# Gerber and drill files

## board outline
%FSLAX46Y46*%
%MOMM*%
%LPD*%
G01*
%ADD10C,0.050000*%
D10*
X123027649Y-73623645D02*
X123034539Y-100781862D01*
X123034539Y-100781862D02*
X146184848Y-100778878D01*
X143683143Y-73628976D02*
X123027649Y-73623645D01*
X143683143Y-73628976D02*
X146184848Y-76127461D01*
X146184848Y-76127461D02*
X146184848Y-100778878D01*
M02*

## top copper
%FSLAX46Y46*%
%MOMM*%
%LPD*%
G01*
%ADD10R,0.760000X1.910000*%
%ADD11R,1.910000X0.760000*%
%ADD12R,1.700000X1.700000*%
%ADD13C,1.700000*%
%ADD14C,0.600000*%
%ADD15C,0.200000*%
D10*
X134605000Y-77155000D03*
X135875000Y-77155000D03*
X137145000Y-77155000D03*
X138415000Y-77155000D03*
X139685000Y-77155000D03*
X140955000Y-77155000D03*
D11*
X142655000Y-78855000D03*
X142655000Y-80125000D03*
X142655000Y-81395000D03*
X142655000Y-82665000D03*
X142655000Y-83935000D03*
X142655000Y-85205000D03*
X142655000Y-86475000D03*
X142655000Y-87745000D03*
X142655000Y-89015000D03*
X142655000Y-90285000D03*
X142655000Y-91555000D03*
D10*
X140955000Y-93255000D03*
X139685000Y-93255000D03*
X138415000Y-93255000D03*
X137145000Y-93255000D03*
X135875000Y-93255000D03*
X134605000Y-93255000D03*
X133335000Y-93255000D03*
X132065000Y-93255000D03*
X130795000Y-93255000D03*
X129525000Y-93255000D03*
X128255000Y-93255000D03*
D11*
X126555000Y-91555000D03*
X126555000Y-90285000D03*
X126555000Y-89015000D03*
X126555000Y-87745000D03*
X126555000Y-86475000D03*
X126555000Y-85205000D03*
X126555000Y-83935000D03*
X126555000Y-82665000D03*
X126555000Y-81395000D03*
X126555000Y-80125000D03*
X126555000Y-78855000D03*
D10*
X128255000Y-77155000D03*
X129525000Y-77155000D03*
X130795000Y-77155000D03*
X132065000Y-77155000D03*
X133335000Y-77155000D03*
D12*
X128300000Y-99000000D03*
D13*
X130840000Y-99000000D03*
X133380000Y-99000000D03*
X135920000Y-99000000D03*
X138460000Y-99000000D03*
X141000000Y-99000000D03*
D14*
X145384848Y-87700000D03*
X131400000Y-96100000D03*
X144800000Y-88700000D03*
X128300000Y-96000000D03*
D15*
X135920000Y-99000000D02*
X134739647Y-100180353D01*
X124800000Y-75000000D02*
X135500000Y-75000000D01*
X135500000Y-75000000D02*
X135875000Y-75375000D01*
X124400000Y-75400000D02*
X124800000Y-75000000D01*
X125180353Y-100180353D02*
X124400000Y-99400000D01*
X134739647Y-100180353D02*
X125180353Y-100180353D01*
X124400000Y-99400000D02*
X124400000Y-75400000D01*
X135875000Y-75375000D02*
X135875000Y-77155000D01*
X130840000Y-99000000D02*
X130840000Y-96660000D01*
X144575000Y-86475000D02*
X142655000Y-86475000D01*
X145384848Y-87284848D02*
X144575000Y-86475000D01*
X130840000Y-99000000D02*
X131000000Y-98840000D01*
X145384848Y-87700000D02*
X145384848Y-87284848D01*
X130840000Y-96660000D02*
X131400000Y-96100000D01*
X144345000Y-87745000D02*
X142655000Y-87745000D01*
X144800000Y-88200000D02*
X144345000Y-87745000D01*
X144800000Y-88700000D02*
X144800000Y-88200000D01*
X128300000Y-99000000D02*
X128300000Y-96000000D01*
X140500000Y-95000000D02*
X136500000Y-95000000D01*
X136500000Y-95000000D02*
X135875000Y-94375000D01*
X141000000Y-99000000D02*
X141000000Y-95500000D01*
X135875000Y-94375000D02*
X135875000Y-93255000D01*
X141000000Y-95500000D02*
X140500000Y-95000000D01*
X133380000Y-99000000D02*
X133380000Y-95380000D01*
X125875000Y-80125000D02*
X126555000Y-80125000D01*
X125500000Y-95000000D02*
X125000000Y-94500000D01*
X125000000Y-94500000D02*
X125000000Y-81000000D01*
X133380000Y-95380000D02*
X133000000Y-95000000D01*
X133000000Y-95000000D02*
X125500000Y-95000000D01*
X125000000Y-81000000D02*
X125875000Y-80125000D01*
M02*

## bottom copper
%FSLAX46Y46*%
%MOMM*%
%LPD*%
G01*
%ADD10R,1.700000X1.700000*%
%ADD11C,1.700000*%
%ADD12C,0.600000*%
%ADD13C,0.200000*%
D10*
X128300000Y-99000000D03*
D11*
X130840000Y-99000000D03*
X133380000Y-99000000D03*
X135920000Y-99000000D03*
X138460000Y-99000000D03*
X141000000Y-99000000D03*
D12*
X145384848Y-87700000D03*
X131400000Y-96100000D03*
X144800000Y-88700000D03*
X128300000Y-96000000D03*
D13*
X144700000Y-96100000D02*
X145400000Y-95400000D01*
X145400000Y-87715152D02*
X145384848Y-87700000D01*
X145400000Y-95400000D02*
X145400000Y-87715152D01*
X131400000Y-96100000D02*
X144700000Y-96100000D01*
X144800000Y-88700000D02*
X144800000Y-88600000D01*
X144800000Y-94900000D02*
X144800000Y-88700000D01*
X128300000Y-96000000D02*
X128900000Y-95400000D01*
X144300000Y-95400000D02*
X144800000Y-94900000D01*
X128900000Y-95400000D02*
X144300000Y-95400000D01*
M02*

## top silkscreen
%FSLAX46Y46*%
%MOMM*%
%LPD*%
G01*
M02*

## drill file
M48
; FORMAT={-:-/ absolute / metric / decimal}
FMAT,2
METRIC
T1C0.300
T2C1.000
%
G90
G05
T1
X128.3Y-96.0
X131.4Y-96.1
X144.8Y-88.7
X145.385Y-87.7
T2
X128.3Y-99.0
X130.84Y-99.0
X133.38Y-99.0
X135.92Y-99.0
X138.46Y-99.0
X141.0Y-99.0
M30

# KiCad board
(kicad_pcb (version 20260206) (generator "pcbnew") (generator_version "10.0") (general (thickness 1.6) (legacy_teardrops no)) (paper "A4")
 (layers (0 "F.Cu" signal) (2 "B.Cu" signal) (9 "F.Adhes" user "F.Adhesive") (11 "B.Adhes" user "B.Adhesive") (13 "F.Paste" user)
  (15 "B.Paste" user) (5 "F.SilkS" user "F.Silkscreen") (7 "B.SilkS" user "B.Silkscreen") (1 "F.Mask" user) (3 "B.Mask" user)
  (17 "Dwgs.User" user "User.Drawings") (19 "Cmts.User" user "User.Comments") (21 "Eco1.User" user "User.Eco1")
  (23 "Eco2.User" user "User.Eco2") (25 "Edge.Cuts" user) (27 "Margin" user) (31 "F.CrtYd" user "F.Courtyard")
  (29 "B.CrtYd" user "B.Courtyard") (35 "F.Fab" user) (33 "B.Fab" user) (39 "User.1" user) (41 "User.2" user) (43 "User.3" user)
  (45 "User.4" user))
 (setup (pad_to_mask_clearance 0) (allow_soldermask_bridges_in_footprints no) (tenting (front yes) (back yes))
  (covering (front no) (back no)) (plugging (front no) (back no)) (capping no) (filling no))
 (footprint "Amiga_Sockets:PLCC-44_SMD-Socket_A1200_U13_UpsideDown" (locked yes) (layer "F.Cu") (at 134.605 85.205)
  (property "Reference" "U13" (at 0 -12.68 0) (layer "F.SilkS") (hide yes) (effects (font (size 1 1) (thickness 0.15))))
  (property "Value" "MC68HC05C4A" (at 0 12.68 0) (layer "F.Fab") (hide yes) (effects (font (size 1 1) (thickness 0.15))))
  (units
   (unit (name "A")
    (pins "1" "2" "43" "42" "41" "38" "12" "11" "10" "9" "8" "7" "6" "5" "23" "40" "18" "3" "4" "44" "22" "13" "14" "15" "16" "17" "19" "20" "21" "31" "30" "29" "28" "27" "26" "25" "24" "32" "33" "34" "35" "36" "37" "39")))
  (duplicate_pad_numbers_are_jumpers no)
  (pad "1" smd rect (at 0 -8.05) (size 0.76 1.91) (layers "F.Cu" "F.Mask" "F.Paste") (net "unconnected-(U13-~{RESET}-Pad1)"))
  (pad "2" smd rect (at 1.27 -8.05) (size 0.76 1.91) (layers "F.Cu" "F.Mask" "F.Paste") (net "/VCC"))
  (pad "3" smd rect (at 2.54 -8.05) (size 0.76 1.91) (layers "F.Cu" "F.Mask" "F.Paste") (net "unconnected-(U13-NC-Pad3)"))
  (pad "4" smd rect (at 3.81 -8.05) (size 0.76 1.91) (layers "F.Cu" "F.Mask" "F.Paste") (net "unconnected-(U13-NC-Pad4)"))
  (pad "5" smd rect (at 5.08 -8.05) (size 0.76 1.91) (layers "F.Cu" "F.Mask" "F.Paste") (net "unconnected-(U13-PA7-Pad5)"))
  (pad "6" smd rect (at 6.35 -8.05) (size 0.76 1.91) (layers "F.Cu" "F.Mask" "F.Paste") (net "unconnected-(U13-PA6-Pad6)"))
  (pad "7" smd rect (at 8.05 -6.35) (size 1.91 0.76) (layers "F.Cu" "F.Mask" "F.Paste") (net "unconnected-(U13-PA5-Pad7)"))
  (pad "8" smd rect (at 8.05 -5.08) (size 1.91 0.76) (layers "F.Cu" "F.Mask" "F.Paste") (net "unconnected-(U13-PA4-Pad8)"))
  (pad "9" smd rect (at 8.05 -3.81) (size 1.91 0.76) (layers "F.Cu" "F.Mask" "F.Paste") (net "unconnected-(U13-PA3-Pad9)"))
  (pad "10" smd rect (at 8.05 -2.54) (size 1.91 0.76) (layers "F.Cu" "F.Mask" "F.Paste") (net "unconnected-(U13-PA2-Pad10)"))
  (pad "11" smd rect (at 8.05 -1.27) (size 1.91 0.76) (layers "F.Cu" "F.Mask" "F.Paste") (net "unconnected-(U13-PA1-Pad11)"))
  (pad "12" smd rect (at 8.05 0) (size 1.91 0.76) (layers "F.Cu" "F.Mask" "F.Paste") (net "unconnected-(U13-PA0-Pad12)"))
  (pad "13" smd rect (at 8.05 1.27) (size 1.91 0.76) (layers "F.Cu" "F.Mask" "F.Paste") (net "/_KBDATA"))
  (pad "14" smd rect (at 8.05 2.54) (size 1.91 0.76) (layers "F.Cu" "F.Mask" "F.Paste") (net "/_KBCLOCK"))
  (pad "15" smd rect (at 8.05 3.81) (size 1.91 0.76) (layers "F.Cu" "F.Mask" "F.Paste") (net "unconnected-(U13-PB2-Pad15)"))
  (pad "16" smd rect (at 8.05 5.08) (size 1.91 0.76) (layers "F.Cu" "F.Mask" "F.Paste") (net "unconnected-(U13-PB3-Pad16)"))
  (pad "17" smd rect (at 8.05 6.35) (size 1.91 0.76) (layers "F.Cu" "F.Mask" "F.Paste") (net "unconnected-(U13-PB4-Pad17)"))
  (pad "18" smd rect (at 6.35 8.05) (size 0.76 1.91) (layers "F.Cu" "F.Mask" "F.Paste") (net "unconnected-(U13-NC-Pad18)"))
  (pad "19" smd rect (at 5.08 8.05) (size 0.76 1.91) (layers "F.Cu" "F.Mask" "F.Paste") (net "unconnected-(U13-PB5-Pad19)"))
  (pad "20" smd rect (at 3.81 8.05) (size 0.76 1.91) (layers "F.Cu" "F.Mask" "F.Paste") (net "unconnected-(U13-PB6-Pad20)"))
  (pad "21" smd rect (at 2.54 8.05) (size 0.76 1.91) (layers "F.Cu" "F.Mask" "F.Paste") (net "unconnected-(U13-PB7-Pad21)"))
  (pad "22" smd rect (at 1.27 8.05) (size 0.76 1.91) (layers "F.Cu" "F.Mask" "F.Paste") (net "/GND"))
  (pad "23" smd rect (at 0 8.05) (size 0.76 1.91) (layers "F.Cu" "F.Mask" "F.Paste") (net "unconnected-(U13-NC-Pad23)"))
  (pad "24" smd rect (at -1.27 8.05) (size 0.76 1.91) (layers "F.Cu" "F.Mask" "F.Paste") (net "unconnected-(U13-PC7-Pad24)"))
  (pad "25" smd rect (at -2.54 8.05) (size 0.76 1.91) (layers "F.Cu" "F.Mask" "F.Paste") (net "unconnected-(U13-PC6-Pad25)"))
  (pad "26" smd rect (at -3.81 8.05) (size 0.76 1.91) (layers "F.Cu" "F.Mask" "F.Paste") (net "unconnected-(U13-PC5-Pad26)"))
  (pad "27" smd rect (at -5.08 8.05) (size 0.76 1.91) (layers "F.Cu" "F.Mask" "F.Paste") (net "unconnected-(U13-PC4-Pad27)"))
  (pad "28" smd rect (at -6.35 8.05) (size 0.76 1.91) (layers "F.Cu" "F.Mask" "F.Paste") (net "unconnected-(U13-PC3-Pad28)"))
  (pad "29" smd rect (at -8.05 6.35) (size 1.91 0.76) (layers "F.Cu" "F.Mask" "F.Paste") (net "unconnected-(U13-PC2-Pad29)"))
  (pad "30" smd rect (at -8.05 5.08) (size 1.91 0.76) (layers "F.Cu" "F.Mask" "F.Paste") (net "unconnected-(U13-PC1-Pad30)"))
  (pad "31" smd rect (at -8.05 3.81) (size 1.91 0.76) (layers "F.Cu" "F.Mask" "F.Paste") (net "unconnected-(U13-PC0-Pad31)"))
  (pad "32" smd rect (at -8.05 2.54) (size 1.91 0.76) (layers "F.Cu" "F.Mask" "F.Paste") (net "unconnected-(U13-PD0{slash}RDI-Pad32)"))
  (pad "33" smd rect (at -8.05 1.27) (size 1.91 0.76) (layers "F.Cu" "F.Mask" "F.Paste") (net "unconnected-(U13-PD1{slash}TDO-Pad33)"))
  (pad "34" smd rect (at -8.05 0) (size 1.91 0.76) (layers "F.Cu" "F.Mask" "F.Paste") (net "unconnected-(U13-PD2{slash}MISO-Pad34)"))
  (pad "35" smd rect (at -8.05 -1.27) (size 1.91 0.76) (layers "F.Cu" "F.Mask" "F.Paste") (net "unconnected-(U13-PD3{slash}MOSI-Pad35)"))
  (pad "36" smd rect (at -8.05 -2.54) (size 1.91 0.76) (layers "F.Cu" "F.Mask" "F.Paste") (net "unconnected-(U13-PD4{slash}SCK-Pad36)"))
  (pad "37" smd rect (at -8.05 -3.81) (size 1.91 0.76) (layers "F.Cu" "F.Mask" "F.Paste") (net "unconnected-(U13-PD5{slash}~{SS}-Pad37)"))
  (pad "38" smd rect (at -8.05 -5.08) (size 1.91 0.76) (layers "F.Cu" "F.Mask" "F.Paste") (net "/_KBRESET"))
  (pad "39" smd rect (at -8.05 -6.35) (size 1.91 0.76) (layers "F.Cu" "F.Mask" "F.Paste") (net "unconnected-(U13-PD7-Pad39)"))
  (pad "40" smd rect (at -6.35 -8.05) (size 0.76 1.91) (layers "F.Cu" "F.Mask" "F.Paste") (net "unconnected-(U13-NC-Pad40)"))
  (pad "41" smd rect (at -5.08 -8.05) (size 0.76 1.91) (layers "F.Cu" "F.Mask" "F.Paste") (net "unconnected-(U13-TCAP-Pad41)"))
  (pad "42" smd rect (at -3.81 -8.05) (size 0.76 1.91) (layers "F.Cu" "F.Mask" "F.Paste") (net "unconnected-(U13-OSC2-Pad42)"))
  (pad "43" smd rect (at -2.54 -8.05) (size 0.76 1.91) (layers "F.Cu" "F.Mask" "F.Paste") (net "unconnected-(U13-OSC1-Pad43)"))
  (pad "44" smd rect (at -1.27 -8.05) (size 0.76 1.91) (layers "F.Cu" "F.Mask" "F.Paste") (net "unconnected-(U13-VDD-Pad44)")))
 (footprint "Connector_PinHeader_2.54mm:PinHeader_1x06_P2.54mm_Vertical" (layer "B.Cu") (at 128.3 99 -90)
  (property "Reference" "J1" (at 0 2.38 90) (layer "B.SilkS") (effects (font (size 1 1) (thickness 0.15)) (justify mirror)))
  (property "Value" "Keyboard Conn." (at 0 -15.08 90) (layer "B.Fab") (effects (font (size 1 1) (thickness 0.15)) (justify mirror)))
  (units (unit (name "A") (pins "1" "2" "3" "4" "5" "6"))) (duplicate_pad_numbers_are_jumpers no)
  (pad "1" thru_hole rect (at 0 0 270) (size 1.7 1.7) (drill 1) (layers "*.Cu" "*.Mask") (remove_unused_layers no) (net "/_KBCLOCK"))
  (pad "2" thru_hole circle (at 0 -2.54 270) (size 1.7 1.7) (drill 1) (layers "*.Cu" "*.Mask") (remove_unused_layers no) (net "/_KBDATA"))
  (pad "3" thru_hole circle (at 0 -5.08 270) (size 1.7 1.7) (drill 1) (layers "*.Cu" "*.Mask") (remove_unused_layers no) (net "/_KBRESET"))
  (pad "4" thru_hole circle (at 0 -7.62 270) (size 1.7 1.7) (drill 1) (layers "*.Cu" "*.Mask") (remove_unused_layers no) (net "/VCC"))
  (pad "5" thru_hole circle (at 0 -10.16 270) (size 1.7 1.7) (drill 1) (layers "*.Cu" "*.Mask") (remove_unused_layers no)
   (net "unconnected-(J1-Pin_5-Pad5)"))
  (pad "6" thru_hole circle (at 0 -12.7 270) (size 1.7 1.7) (drill 1) (layers "*.Cu" "*.Mask") (remove_unused_layers no) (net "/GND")))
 (gr_line (start 123.027649 73.623645) (end 123.034539 100.781862) (stroke (width 0.05) (type default)) (layer "Edge.Cuts"))
 (gr_line (start 123.034539 100.781862) (end 146.184848 100.778878) (stroke (width 0.05) (type default)) (layer "Edge.Cuts"))
 (gr_line (start 143.683143 73.628976) (end 123.027649 73.623645) (stroke (width 0.05) (type default)) (layer "Edge.Cuts"))
 (gr_line (start 143.683143 73.628976) (end 146.184848 76.127461) (stroke (width 0.05) (type default)) (layer "Edge.Cuts"))
 (gr_line (start 146.184848 76.127461) (end 146.184848 100.778878) (stroke (width 0.05) (type default)) (layer "Edge.Cuts"))
 (segment (start 135.92 99) (end 134.739647 100.180353) (width 0.2) (layer "F.Cu") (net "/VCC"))
 (segment (start 124.8 75) (end 135.5 75) (width 0.2) (layer "F.Cu") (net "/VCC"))
 (segment (start 135.5 75) (end 135.875 75.375) (width 0.2) (layer "F.Cu") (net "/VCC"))
 (segment (start 124.4 75.4) (end 124.8 75) (width 0.2) (layer "F.Cu") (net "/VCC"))
 (segment (start 125.180353 100.180353) (end 124.4 99.4) (width 0.2) (layer "F.Cu") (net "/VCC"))
 (segment (start 134.739647 100.180353) (end 125.180353 100.180353) (width 0.2) (layer "F.Cu") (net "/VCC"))
 (segment (start 124.4 99.4) (end 124.4 75.4) (width 0.2) (layer "F.Cu") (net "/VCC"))
 (segment (start 135.875 75.375) (end 135.875 77.155) (width 0.2) (layer "F.Cu") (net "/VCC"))
 (segment (start 130.84 99) (end 130.84 96.66) (width 0.2) (layer "F.Cu") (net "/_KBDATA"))
 (segment (start 144.575 86.475) (end 142.655 86.475) (width 0.2) (layer "F.Cu") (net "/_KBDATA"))
 (segment (start 145.384848 87.284848) (end 144.575 86.475) (width 0.2) (layer "F.Cu") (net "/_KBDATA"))
 (segment (start 130.84 99) (end 131 98.84) (width 0.2) (layer "F.Cu") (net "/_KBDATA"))
 (segment (start 145.384848 87.7) (end 145.384848 87.284848) (width 0.2) (layer "F.Cu") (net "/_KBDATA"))
 (segment (start 130.84 96.66) (end 131.4 96.1) (width 0.2) (layer "F.Cu") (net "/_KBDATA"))
 (via (at 145.384848 87.7) (size 0.6) (drill 0.3) (layers "F.Cu" "B.Cu") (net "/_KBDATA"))
 (via (at 131.4 96.1) (size 0.6) (drill 0.3) (layers "F.Cu" "B.Cu") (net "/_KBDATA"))
 (segment (start 144.7 96.1) (end 145.4 95.4) (width 0.2) (layer "B.Cu") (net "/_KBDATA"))
 (segment (start 145.4 87.715152) (end 145.384848 87.7) (width 0.2) (layer "B.Cu") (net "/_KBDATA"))
 (segment (start 145.4 95.4) (end 145.4 87.715152) (width 0.2) (layer "B.Cu") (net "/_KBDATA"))
 (segment (start 131.4 96.1) (end 144.7 96.1) (width 0.2) (layer "B.Cu") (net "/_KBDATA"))
 (segment (start 144.345 87.745) (end 142.655 87.745) (width 0.2) (layer "F.Cu") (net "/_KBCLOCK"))
 (segment (start 144.8 88.2) (end 144.345 87.745) (width 0.2) (layer "F.Cu") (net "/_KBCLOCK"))
 (segment (start 144.8 88.7) (end 144.8 88.2) (width 0.2) (layer "F.Cu") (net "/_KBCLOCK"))
 (segment (start 128.3 99) (end 128.3 96) (width 0.2) (layer "F.Cu") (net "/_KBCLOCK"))
 (via (at 144.8 88.7) (size 0.6) (drill 0.3) (layers "F.Cu" "B.Cu") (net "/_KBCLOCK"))
 (via (at 128.3 96) (size 0.6) (drill 0.3) (layers "F.Cu" "B.Cu") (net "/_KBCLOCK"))
 (segment (start 144.8 88.7) (end 144.8 88.6) (width 0.2) (layer "B.Cu") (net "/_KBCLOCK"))
 (segment (start 144.8 94.9) (end 144.8 88.7) (width 0.2) (layer "B.Cu") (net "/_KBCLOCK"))
 (segment (start 128.3 96) (end 128.9 95.4) (width 0.2) (layer "B.Cu") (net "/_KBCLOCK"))
 (segment (start 144.3 95.4) (end 144.8 94.9) (width 0.2) (layer "B.Cu") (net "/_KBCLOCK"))
 (segment (start 128.9 95.4) (end 144.3 95.4) (width 0.2) (layer "B.Cu") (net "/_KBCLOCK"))
 (segment (start 140.5 95) (end 136.5 95) (width 0.2) (layer "F.Cu") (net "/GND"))
 (segment (start 136.5 95) (end 135.875 94.375) (width 0.2) (layer "F.Cu") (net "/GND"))
 (segment (start 141 99) (end 141 95.5) (width 0.2) (layer "F.Cu") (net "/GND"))
 (segment (start 135.875 94.375) (end 135.875 93.255) (width 0.2) (layer "F.Cu") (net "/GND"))
 (segment (start 141 95.5) (end 140.5 95) (width 0.2) (layer "F.Cu") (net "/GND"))
 (segment (start 133.38 99) (end 133.38 95.38) (width 0.2) (layer "F.Cu") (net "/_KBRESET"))
 (segment (start 125.875 80.125) (end 126.555 80.125) (width 0.2) (layer "F.Cu") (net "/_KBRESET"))
 (segment (start 125.5 95) (end 125 94.5) (width 0.2) (layer "F.Cu") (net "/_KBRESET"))
 (segment (start 125 94.5) (end 125 81) (width 0.2) (layer "F.Cu") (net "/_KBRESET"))
 (segment (start 133.38 95.38) (end 133 95) (width 0.2) (layer "F.Cu") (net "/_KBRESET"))
 (segment (start 133 95) (end 125.5 95) (width 0.2) (layer "F.Cu") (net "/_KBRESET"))
 (segment (start 125 81) (end 125.875 80.125) (width 0.2) (layer "F.Cu") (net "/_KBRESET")))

